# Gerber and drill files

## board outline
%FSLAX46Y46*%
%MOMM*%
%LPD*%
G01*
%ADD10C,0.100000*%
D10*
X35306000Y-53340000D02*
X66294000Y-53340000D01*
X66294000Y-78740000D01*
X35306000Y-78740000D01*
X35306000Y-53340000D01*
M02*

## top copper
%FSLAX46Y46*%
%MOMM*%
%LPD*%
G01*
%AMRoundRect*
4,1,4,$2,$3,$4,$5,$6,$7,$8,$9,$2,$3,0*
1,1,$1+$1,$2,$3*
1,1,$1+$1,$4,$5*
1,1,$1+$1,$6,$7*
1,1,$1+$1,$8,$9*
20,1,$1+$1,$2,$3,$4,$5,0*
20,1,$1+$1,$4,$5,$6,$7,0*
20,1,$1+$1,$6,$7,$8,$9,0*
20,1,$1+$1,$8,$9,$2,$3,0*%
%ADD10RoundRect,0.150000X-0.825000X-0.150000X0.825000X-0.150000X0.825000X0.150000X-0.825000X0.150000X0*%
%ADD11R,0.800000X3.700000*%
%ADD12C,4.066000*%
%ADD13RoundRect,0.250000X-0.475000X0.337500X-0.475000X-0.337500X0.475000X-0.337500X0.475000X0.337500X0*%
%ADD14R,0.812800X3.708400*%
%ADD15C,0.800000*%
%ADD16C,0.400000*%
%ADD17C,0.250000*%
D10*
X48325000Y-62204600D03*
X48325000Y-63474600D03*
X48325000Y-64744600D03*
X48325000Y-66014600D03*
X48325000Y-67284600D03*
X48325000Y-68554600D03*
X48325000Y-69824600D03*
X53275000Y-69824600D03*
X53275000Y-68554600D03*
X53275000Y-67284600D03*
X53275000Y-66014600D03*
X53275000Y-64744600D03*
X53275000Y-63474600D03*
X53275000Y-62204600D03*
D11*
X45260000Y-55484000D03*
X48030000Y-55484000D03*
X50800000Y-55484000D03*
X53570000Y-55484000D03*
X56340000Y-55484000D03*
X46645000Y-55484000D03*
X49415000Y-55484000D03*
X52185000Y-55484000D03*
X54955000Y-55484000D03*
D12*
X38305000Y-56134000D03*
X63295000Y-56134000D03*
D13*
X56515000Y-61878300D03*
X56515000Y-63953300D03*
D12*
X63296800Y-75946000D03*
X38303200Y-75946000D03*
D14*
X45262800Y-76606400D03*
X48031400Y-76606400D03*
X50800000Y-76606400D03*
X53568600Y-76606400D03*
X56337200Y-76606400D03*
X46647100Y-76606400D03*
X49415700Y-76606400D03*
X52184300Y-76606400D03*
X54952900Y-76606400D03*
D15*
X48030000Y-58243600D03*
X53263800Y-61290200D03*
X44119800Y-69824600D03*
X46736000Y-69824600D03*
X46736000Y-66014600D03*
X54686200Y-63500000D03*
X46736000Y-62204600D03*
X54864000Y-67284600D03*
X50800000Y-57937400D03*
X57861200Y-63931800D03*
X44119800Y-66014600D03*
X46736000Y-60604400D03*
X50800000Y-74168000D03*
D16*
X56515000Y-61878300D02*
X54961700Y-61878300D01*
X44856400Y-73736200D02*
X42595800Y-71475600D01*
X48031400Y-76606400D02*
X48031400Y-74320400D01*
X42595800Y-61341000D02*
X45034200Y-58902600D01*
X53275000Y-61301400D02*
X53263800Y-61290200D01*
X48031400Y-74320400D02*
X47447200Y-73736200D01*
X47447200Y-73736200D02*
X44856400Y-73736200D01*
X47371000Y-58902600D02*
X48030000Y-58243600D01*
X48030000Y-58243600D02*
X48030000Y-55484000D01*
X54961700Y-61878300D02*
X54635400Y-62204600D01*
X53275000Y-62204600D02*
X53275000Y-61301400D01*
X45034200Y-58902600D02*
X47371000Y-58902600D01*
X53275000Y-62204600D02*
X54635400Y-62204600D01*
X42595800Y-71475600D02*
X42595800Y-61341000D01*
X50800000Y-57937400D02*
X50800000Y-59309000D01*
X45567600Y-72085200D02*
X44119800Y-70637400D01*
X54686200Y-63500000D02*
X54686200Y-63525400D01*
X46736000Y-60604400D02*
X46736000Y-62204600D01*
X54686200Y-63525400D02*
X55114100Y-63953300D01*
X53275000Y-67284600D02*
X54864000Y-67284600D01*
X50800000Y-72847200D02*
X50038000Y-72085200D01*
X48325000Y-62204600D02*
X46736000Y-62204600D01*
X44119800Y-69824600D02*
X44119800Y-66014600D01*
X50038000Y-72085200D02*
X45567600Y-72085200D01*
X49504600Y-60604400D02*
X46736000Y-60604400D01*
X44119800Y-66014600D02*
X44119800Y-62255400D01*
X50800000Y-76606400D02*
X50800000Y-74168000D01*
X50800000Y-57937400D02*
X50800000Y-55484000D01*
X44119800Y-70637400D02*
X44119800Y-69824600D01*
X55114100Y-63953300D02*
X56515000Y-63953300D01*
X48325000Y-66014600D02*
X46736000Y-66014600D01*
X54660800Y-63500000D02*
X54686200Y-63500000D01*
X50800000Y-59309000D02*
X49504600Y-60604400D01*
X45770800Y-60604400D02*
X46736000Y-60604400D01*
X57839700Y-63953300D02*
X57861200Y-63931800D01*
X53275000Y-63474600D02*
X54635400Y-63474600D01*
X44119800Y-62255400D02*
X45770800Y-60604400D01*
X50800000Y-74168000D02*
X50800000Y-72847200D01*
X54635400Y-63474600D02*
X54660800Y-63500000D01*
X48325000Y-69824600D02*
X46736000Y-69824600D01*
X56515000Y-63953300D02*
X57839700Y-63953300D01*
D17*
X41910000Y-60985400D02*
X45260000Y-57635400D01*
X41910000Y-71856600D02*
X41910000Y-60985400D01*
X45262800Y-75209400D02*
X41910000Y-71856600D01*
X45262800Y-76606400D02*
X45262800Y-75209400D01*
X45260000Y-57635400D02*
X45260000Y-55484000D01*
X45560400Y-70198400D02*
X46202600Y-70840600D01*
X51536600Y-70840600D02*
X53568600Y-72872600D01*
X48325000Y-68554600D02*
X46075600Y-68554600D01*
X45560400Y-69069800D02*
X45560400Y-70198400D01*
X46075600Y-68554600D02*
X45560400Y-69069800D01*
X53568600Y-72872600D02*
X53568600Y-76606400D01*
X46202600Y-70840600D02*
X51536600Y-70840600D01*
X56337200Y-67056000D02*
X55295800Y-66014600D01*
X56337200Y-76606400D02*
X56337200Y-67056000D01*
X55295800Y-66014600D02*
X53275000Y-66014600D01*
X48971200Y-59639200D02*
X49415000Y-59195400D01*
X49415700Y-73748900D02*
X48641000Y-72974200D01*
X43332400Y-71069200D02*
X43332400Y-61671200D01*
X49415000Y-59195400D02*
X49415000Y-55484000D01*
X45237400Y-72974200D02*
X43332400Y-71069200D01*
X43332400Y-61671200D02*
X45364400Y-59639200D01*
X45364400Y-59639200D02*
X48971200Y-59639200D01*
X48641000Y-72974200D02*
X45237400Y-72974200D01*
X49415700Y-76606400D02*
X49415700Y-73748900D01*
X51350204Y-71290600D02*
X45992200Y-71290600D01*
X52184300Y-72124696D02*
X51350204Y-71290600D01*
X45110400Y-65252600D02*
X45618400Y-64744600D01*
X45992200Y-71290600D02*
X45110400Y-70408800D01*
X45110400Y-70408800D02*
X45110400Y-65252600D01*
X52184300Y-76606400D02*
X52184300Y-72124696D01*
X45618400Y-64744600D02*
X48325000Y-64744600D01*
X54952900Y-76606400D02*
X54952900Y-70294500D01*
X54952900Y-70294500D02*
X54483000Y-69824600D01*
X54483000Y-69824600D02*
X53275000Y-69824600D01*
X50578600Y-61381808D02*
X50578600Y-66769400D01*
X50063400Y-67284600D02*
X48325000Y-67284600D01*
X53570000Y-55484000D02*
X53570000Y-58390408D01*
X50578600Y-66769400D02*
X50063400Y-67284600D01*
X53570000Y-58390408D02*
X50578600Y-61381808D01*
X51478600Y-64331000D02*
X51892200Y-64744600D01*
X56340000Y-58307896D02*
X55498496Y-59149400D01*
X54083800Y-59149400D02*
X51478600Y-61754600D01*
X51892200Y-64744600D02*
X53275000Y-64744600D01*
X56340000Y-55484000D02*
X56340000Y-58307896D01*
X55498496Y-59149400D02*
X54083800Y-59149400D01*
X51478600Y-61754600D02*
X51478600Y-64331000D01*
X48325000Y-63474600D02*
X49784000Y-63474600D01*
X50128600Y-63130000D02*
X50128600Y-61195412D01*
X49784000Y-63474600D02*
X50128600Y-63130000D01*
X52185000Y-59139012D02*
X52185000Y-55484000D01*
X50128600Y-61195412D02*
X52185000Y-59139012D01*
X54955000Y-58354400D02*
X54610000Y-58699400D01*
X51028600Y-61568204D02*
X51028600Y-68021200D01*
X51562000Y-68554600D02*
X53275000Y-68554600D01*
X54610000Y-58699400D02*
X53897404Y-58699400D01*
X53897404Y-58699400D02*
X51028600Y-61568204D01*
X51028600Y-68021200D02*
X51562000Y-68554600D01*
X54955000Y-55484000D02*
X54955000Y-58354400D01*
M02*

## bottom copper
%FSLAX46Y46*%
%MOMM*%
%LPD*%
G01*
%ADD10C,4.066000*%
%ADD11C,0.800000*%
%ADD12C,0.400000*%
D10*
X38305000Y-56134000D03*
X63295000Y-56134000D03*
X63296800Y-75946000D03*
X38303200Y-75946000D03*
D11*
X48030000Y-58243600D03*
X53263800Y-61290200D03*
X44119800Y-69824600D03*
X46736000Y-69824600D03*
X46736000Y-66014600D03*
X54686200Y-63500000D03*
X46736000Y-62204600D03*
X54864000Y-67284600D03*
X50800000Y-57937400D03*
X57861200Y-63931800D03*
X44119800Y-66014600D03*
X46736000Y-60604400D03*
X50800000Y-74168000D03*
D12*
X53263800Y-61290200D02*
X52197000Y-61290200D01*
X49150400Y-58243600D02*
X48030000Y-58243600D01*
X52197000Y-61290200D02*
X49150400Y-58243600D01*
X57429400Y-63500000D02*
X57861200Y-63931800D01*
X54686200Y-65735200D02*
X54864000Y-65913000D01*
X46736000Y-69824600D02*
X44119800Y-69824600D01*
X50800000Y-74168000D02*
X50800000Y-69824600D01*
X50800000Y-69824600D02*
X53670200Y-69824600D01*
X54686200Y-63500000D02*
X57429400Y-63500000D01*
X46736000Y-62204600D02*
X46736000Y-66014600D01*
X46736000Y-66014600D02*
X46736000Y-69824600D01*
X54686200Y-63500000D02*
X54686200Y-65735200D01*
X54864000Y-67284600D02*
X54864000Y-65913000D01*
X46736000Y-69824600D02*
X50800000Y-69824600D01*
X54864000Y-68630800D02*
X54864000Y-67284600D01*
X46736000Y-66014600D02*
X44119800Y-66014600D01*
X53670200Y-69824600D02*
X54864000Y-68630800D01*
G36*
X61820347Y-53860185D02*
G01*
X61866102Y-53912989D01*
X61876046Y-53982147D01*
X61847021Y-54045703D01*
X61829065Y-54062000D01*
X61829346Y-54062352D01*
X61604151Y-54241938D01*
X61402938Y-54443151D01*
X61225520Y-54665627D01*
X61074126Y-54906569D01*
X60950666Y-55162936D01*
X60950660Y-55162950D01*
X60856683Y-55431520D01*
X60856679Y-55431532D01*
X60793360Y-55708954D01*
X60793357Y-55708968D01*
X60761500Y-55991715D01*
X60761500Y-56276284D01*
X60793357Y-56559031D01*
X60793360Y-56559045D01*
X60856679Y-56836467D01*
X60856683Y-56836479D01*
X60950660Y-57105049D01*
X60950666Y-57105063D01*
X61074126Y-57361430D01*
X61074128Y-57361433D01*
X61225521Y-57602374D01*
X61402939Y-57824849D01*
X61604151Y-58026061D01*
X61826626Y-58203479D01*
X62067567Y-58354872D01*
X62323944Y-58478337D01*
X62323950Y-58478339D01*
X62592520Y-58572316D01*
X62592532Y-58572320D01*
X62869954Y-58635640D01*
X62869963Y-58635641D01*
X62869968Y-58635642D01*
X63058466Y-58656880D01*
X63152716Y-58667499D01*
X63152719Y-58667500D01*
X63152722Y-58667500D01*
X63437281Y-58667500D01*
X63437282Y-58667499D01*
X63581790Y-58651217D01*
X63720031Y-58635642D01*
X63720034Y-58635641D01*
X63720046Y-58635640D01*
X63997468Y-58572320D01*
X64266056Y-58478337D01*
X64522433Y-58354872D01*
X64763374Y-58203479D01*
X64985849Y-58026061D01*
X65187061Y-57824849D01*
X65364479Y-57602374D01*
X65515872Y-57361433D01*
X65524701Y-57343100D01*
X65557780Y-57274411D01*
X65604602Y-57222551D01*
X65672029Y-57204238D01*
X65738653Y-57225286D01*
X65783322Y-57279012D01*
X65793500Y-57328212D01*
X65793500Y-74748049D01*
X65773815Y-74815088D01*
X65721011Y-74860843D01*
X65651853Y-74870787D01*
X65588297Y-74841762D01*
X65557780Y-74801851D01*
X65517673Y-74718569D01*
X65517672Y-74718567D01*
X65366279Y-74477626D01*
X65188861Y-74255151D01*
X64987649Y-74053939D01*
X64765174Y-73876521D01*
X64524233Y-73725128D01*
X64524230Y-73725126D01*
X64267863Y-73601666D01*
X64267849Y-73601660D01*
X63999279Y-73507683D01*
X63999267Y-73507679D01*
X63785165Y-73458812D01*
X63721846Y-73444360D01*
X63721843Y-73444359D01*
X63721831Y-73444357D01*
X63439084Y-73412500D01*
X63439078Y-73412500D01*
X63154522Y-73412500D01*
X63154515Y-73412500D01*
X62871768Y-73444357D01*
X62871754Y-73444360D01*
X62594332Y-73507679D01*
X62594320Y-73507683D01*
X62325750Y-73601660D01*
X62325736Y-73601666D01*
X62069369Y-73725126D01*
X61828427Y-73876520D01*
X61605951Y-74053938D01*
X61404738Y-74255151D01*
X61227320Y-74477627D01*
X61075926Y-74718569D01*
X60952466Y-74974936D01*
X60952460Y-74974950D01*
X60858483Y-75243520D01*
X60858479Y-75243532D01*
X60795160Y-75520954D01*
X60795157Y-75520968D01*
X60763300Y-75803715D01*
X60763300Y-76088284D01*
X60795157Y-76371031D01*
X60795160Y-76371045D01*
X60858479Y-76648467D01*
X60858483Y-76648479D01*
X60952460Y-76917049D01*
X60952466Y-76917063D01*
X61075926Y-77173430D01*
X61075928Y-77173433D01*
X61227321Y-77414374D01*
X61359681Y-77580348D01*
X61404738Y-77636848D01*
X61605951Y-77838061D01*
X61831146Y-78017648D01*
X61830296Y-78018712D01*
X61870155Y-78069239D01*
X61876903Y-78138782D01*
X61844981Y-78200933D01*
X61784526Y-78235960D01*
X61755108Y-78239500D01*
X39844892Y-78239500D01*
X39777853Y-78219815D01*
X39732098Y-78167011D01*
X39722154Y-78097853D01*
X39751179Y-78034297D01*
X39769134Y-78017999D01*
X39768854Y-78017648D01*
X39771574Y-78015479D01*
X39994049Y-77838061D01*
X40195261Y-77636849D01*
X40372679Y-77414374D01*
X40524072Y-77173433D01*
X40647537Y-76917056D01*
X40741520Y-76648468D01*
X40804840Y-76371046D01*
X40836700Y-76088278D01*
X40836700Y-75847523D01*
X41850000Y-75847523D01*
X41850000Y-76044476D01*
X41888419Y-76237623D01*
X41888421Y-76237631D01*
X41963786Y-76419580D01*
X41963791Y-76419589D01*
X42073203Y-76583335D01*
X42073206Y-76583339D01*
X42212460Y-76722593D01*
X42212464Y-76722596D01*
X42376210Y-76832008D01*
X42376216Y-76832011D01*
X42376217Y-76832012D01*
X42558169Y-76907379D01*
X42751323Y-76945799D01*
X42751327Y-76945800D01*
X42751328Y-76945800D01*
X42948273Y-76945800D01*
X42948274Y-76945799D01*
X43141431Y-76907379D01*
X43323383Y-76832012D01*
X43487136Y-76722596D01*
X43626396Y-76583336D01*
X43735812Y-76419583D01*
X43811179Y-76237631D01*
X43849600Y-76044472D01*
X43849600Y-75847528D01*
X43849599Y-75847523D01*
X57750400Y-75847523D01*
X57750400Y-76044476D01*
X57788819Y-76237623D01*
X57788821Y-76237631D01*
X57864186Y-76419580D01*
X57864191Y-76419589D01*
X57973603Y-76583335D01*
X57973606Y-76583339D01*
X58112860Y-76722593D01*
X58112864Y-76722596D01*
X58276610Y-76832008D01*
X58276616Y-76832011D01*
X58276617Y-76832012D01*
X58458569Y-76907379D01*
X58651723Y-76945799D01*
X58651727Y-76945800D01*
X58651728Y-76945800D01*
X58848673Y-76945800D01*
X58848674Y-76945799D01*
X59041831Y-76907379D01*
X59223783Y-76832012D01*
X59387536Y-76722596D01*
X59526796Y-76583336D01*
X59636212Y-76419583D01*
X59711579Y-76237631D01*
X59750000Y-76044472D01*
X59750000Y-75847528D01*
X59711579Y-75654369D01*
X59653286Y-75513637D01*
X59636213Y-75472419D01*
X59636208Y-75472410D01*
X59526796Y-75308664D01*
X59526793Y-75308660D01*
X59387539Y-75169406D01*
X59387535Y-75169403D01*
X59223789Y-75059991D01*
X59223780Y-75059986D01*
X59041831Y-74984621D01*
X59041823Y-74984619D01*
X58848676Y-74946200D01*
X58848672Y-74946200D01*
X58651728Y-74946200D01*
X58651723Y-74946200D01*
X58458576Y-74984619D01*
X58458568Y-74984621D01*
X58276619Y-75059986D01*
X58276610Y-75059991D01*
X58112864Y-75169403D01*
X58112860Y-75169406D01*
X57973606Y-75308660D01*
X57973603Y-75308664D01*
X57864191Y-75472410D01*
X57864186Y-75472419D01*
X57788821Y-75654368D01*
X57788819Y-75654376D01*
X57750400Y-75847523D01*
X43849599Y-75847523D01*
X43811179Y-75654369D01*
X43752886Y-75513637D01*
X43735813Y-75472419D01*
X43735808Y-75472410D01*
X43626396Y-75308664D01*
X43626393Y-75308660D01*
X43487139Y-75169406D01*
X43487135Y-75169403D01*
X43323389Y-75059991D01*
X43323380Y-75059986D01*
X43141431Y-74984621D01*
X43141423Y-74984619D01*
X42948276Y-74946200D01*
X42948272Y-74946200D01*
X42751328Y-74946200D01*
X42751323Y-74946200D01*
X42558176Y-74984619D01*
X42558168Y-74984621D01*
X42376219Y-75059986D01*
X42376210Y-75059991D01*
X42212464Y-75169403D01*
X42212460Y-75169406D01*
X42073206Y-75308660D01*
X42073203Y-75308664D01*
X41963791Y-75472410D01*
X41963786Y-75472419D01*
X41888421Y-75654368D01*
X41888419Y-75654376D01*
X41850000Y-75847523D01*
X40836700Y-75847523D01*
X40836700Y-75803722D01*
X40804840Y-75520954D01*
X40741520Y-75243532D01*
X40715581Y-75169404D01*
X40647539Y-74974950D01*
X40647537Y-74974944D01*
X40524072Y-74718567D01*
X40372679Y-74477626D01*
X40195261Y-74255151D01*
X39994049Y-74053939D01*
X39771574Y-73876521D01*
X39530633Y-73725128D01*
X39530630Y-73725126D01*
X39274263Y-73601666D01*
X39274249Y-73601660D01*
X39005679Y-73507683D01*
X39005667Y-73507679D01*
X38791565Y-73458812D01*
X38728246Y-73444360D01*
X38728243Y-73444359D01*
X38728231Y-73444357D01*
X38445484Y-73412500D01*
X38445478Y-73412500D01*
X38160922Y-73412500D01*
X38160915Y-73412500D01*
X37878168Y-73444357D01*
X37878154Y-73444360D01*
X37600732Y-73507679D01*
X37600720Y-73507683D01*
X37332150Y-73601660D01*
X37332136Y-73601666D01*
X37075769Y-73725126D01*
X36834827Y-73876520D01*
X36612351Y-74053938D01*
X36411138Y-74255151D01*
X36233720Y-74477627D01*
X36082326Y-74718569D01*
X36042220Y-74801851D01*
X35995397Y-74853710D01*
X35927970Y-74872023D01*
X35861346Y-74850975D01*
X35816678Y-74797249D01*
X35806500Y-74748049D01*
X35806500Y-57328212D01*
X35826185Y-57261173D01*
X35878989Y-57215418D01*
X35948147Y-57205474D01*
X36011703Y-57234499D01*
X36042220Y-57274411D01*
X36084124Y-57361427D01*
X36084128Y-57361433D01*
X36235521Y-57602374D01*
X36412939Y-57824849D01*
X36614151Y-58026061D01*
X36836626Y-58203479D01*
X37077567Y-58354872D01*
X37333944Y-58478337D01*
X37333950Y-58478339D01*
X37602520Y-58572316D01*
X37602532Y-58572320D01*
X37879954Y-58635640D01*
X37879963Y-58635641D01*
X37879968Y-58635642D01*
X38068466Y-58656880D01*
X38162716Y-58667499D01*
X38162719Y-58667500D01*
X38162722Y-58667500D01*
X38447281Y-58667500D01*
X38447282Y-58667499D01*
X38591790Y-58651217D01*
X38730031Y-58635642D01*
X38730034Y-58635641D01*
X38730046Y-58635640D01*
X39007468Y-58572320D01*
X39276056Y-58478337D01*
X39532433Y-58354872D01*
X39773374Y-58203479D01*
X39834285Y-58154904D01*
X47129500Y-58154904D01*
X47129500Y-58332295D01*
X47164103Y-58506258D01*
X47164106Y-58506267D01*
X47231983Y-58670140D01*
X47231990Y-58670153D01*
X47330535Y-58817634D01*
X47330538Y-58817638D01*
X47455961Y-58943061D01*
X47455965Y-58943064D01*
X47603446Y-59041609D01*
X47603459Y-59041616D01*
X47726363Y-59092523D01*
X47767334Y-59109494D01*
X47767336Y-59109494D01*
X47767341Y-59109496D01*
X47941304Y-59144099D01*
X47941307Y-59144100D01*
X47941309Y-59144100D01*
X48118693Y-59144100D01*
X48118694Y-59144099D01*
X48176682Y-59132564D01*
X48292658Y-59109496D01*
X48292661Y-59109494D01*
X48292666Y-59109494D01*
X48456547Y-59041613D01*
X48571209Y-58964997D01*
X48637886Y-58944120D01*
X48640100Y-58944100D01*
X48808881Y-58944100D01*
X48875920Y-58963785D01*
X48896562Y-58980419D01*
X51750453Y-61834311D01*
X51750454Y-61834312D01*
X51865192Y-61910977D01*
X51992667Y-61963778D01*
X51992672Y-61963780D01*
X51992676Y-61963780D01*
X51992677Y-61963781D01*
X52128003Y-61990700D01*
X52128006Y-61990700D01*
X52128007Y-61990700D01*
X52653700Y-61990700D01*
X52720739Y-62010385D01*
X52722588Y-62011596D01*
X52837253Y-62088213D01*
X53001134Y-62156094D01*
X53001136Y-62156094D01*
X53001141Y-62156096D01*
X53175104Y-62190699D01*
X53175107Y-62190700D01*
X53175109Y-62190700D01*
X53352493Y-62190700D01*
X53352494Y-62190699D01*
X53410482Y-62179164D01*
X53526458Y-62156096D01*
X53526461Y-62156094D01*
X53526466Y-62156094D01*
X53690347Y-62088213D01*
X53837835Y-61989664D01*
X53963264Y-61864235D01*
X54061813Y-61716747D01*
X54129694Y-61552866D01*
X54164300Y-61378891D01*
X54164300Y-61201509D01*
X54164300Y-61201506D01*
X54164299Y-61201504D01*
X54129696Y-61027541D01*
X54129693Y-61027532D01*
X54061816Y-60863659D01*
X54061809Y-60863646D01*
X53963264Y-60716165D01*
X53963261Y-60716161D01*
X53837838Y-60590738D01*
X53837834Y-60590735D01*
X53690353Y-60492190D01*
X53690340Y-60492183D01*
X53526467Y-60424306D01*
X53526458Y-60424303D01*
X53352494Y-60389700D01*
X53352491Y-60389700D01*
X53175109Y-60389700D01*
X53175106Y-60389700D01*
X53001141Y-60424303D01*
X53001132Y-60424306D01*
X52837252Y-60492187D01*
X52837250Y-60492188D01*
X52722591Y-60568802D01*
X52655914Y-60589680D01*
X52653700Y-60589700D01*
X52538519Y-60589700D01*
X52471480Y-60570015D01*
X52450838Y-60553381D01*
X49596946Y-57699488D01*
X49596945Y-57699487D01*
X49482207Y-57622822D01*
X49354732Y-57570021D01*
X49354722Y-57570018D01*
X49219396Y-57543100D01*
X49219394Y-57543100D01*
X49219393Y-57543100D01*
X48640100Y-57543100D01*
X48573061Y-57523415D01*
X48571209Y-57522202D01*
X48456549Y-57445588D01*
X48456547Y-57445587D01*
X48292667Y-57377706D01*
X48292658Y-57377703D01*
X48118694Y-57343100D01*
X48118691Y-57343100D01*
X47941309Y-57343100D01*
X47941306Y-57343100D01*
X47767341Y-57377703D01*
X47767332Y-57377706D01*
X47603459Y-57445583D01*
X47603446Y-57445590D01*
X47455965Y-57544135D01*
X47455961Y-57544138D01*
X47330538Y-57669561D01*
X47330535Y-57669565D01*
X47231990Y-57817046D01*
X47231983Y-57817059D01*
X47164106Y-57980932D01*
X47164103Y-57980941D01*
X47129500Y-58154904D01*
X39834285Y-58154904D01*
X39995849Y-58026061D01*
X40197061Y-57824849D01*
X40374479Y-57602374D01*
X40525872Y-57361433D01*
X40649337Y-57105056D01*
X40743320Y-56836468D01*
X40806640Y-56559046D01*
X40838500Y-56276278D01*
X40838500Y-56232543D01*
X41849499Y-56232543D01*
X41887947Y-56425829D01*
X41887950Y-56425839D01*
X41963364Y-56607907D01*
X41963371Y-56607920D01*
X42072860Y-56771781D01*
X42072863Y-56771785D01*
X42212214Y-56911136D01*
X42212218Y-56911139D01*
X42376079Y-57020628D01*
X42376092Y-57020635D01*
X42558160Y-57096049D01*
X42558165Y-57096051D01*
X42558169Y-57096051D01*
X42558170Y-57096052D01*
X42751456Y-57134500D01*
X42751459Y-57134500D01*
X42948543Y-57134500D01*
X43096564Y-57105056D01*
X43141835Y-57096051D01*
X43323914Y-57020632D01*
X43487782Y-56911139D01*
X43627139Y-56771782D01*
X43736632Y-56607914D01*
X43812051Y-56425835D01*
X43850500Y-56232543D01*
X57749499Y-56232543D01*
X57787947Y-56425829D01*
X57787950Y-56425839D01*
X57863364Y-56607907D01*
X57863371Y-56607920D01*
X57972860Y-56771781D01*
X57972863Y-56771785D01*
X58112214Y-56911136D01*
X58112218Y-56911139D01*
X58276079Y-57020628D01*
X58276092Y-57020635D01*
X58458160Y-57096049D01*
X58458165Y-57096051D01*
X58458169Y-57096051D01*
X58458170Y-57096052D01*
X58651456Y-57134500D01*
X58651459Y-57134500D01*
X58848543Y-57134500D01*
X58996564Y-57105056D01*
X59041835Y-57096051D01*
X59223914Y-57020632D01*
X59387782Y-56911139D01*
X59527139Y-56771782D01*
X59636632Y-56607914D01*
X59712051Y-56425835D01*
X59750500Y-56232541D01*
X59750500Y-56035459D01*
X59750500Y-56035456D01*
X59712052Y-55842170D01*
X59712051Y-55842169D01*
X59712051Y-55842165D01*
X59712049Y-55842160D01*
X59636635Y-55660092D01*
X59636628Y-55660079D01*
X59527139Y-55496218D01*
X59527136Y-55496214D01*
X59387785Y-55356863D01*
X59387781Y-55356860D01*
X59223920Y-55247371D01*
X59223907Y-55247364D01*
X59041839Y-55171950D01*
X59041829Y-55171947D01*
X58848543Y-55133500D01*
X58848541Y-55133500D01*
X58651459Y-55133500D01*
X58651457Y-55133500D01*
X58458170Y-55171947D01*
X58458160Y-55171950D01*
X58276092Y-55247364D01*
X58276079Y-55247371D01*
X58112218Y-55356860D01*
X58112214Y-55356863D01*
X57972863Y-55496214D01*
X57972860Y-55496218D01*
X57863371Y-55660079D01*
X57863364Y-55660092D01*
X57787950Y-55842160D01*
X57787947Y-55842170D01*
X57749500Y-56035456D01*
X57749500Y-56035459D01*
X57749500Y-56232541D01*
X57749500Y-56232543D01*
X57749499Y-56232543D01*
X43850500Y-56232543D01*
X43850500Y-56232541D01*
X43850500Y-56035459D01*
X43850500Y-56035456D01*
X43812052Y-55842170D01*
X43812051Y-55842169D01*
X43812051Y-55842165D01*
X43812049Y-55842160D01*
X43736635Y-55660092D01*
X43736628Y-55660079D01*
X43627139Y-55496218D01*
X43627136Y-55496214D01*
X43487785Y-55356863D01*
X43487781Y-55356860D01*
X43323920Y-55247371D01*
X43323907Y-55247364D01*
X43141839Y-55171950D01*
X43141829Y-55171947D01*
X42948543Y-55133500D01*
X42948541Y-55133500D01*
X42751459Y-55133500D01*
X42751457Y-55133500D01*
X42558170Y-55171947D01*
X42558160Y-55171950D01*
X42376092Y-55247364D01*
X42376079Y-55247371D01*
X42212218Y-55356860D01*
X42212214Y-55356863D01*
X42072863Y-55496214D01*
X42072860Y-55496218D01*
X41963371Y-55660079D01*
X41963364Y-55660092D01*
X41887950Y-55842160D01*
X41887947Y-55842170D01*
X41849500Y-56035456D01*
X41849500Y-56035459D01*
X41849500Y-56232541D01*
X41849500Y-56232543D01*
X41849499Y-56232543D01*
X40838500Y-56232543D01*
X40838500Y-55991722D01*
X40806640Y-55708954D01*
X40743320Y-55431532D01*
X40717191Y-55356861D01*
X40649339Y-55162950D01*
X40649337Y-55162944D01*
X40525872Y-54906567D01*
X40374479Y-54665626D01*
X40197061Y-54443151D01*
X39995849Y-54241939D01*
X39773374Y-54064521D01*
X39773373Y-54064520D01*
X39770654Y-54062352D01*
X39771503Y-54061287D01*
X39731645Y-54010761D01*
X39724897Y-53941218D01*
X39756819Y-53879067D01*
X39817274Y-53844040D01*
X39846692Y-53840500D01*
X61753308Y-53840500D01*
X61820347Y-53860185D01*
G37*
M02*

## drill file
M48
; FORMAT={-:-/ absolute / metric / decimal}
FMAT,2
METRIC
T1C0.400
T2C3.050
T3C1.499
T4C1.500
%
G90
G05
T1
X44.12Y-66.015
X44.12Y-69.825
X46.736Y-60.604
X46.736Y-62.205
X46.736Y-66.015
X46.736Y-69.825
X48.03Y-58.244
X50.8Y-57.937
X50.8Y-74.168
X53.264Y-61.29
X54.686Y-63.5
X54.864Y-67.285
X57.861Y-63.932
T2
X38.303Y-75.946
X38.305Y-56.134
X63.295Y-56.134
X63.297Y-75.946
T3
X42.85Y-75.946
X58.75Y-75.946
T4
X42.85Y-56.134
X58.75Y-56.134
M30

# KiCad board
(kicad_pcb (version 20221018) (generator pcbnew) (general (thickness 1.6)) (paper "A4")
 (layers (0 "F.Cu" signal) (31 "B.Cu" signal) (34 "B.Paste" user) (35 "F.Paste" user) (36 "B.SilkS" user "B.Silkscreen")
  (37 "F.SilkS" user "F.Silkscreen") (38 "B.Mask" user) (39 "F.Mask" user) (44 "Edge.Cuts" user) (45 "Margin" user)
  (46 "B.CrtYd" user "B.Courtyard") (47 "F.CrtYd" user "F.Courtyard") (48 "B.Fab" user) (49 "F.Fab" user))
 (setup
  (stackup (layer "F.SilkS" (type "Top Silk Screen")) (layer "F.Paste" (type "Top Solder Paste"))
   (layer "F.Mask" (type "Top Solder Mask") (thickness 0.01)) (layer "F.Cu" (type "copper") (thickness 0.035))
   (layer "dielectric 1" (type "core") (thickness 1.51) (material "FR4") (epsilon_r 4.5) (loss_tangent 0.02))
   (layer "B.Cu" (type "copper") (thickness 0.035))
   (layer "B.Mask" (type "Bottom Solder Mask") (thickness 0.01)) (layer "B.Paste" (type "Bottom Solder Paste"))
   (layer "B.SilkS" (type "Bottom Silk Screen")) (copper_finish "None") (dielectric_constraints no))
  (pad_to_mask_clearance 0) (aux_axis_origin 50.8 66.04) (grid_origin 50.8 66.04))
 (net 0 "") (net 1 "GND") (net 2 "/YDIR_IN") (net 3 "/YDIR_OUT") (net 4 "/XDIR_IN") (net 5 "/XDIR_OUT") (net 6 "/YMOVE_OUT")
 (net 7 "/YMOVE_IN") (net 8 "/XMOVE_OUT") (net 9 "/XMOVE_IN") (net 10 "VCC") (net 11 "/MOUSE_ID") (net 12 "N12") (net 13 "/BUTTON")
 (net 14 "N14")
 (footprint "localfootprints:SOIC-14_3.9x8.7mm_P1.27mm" (layer "F.Cu") (at 50.8 66.0146)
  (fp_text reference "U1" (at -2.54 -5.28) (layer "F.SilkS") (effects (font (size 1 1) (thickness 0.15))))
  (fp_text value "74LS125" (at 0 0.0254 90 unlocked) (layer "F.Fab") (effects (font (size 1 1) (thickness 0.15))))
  (pad "1" smd roundrect (at -2.475 -3.81) (size 1.95 0.6) (layers "F.Cu" "F.Paste" "F.Mask") (roundrect_rratio 0.25) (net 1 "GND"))
  (pad "2" smd roundrect (at -2.475 -2.54) (size 1.95 0.6) (layers "F.Cu" "F.Paste" "F.Mask") (roundrect_rratio 0.25) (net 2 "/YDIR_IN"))
  (pad "3" smd roundrect (at -2.475 -1.27) (size 1.95 0.6) (layers "F.Cu" "F.Paste" "F.Mask") (roundrect_rratio 0.25) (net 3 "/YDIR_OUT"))
  (pad "4" smd roundrect (at -2.475 0) (size 1.95 0.6) (layers "F.Cu" "F.Paste" "F.Mask") (roundrect_rratio 0.25) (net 1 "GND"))
  (pad "5" smd roundrect (at -2.475 1.27) (size 1.95 0.6) (layers "F.Cu" "F.Paste" "F.Mask") (roundrect_rratio 0.25) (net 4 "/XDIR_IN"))
  (pad "6" smd roundrect (at -2.475 2.54) (size 1.95 0.6) (layers "F.Cu" "F.Paste" "F.Mask") (roundrect_rratio 0.25) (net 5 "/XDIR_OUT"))
  (pad "7" smd roundrect (at -2.475 3.81) (size 1.95 0.6) (layers "F.Cu" "F.Paste" "F.Mask") (roundrect_rratio 0.25) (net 1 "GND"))
  (pad "8" smd roundrect (at 2.475 3.81) (size 1.95 0.6) (layers "F.Cu" "F.Paste" "F.Mask") (roundrect_rratio 0.25) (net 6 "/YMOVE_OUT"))
  (pad "9" smd roundrect (at 2.475 2.54) (size 1.95 0.6) (layers "F.Cu" "F.Paste" "F.Mask") (roundrect_rratio 0.25) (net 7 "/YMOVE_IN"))
  (pad "10" smd roundrect (at 2.475 1.27) (size 1.95 0.6) (layers "F.Cu" "F.Paste" "F.Mask") (roundrect_rratio 0.25) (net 1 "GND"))
  (pad "11" smd roundrect (at 2.475 0) (size 1.95 0.6) (layers "F.Cu" "F.Paste" "F.Mask") (roundrect_rratio 0.25) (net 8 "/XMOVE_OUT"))
  (pad "12" smd roundrect (at 2.475 -1.27) (size 1.95 0.6) (layers "F.Cu" "F.Paste" "F.Mask") (roundrect_rratio 0.25) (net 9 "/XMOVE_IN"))
  (pad "13" smd roundrect (at 2.475 -2.54) (size 1.95 0.6) (layers "F.Cu" "F.Paste" "F.Mask") (roundrect_rratio 0.25) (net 1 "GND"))
  (pad "14" smd roundrect (at 2.475 -3.81) (size 1.95 0.6) (layers "F.Cu" "F.Paste" "F.Mask") (roundrect_rratio 0.25) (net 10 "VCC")))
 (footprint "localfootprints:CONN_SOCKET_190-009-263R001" (layer "F.Cu") (at 50.8 56.134)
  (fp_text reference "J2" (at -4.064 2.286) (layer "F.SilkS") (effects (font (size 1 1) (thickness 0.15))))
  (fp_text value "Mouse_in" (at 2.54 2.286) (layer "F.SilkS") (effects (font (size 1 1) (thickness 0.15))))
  (pad "" np_thru_hole circle (at -7.95 0) (size 1.5 1.5) (drill 1.5) (layers "*.Cu" "*.Mask"))
  (pad "" np_thru_hole circle (at 7.95 0) (size 1.5 1.5) (drill 1.5) (layers "*.Cu" "*.Mask"))
  (pad "1" smd rect (at -5.54 -0.65) (size 0.8 3.7) (layers "F.Cu" "F.Paste" "F.Mask") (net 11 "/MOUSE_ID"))
  (pad "2" smd rect (at -2.77 -0.65) (size 0.8 3.7) (layers "F.Cu" "F.Paste" "F.Mask") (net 10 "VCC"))
  (pad "3" smd rect (at 0 -0.65) (size 0.8 3.7) (layers "F.Cu" "F.Paste" "F.Mask") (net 1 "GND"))
  (pad "4" smd rect (at 2.77 -0.65) (size 0.8 3.7) (layers "F.Cu" "F.Paste" "F.Mask") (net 4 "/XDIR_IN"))
  (pad "5" smd rect (at 5.54 -0.65) (size 0.8 3.7) (layers "F.Cu" "F.Paste" "F.Mask") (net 9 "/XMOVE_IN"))
  (pad "6" smd rect (at -4.155 -0.65) (size 0.8 3.7) (layers "F.Cu" "F.Paste" "F.Mask") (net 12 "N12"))
  (pad "7" smd rect (at -1.385 -0.65) (size 0.8 3.7) (layers "F.Cu" "F.Paste" "F.Mask") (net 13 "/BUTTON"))
  (pad "8" smd rect (at 1.385 -0.65) (size 0.8 3.7) (layers "F.Cu" "F.Paste" "F.Mask") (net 2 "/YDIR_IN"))
  (pad "9" smd rect (at 4.155 -0.65) (size 0.8 3.7) (layers "F.Cu" "F.Paste" "F.Mask") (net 7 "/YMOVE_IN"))
  (pad "S1" thru_hole circle (at -12.495 0) (size 4.066 4.066) (drill 3.05) (layers "*.Cu" "*.Mask"))
  (pad "S2" thru_hole circle (at 12.495 0) (size 4.066 4.066) (drill 3.05) (layers "*.Cu" "*.Mask")))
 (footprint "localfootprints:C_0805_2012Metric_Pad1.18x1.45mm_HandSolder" (layer "F.Cu") (at 56.515 62.9158 -90)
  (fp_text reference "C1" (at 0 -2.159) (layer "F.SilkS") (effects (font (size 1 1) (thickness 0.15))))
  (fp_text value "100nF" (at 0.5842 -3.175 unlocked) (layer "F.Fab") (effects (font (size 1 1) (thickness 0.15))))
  (pad "1" smd roundrect (at -1.0375 0 270) (size 1.175 1.45) (layers "F.Cu" "F.Paste" "F.Mask") (roundrect_rratio 0.2127659574)
   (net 10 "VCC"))
  (pad "2" smd roundrect (at 1.0375 0 270) (size 1.175 1.45) (layers "F.Cu" "F.Paste" "F.Mask") (roundrect_rratio 0.2127659574)
   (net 1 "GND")))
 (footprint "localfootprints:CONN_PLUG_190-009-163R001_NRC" (layer "F.Cu") (at 50.8 75.946 180)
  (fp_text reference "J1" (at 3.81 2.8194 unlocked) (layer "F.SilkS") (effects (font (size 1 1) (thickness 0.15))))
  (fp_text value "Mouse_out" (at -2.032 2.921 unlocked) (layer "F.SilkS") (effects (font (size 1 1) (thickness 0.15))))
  (pad "" thru_hole circle (at -12.4968 0 180) (size 4.066 4.066) (drill 3.05) (layers "*.Cu" "*.Mask"))
  (pad "" np_thru_hole circle (at -7.9502 0 180) (size 1.4986 1.4986) (drill 1.4986) (layers))
  (pad "" np_thru_hole circle (at 7.9502 0 180) (size 1.4986 1.4986) (drill 1.4986) (layers))
  (pad "" thru_hole circle (at 12.4968 0 180) (size 4.066 4.066) (drill 3.05) (layers "*.Cu" "*.Mask"))
  (pad "1" smd rect (at 5.5372 -0.6604 180) (size 0.8128 3.7084) (layers "F.Cu" "F.Paste" "F.Mask") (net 11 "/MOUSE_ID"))
  (pad "2" smd rect (at 2.7686 -0.6604 180) (size 0.8128 3.7084) (layers "F.Cu" "F.Paste" "F.Mask") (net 10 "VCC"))
  (pad "3" smd rect (at 0 -0.6604 180) (size 0.8128 3.7084) (layers "F.Cu" "F.Paste" "F.Mask") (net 1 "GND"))
  (pad "4" smd rect (at -2.7686 -0.6604 180) (size 0.8128 3.7084) (layers "F.Cu" "F.Paste" "F.Mask") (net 5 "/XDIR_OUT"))
  (pad "5" smd rect (at -5.5372 -0.6604 180) (size 0.8128 3.7084) (layers "F.Cu" "F.Paste" "F.Mask") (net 8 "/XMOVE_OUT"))
  (pad "6" smd rect (at 4.1529 -0.6604 180) (size 0.8128 3.7084) (layers "F.Cu" "F.Paste" "F.Mask") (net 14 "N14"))
  (pad "7" smd rect (at 1.3843 -0.6604 180) (size 0.8128 3.7084) (layers "F.Cu" "F.Paste" "F.Mask") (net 13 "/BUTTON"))
  (pad "8" smd rect (at -1.3843 -0.6604 180) (size 0.8128 3.7084) (layers "F.Cu" "F.Paste" "F.Mask") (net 3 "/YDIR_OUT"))
  (pad "9" smd rect (at -4.1529 -0.6604 180) (size 0.8128 3.7084) (layers "F.Cu" "F.Paste" "F.Mask") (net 6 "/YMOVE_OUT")))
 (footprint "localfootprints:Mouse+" (layer "B.Cu") (at 50.8 66.04 180)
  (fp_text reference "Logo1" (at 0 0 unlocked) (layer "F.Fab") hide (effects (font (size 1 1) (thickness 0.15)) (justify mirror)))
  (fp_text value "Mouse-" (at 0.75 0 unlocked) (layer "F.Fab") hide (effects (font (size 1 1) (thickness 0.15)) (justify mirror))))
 (gr_rect (start 35.306 53.34) (end 66.294 78.74) (stroke (width 0.1) (type default)) (fill none) (layer "Edge.Cuts"))
 (segment (start 56.515 61.8783) (end 54.9617 61.8783) (width 0.4) (layer "F.Cu") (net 10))
 (segment (start 44.8564 73.7362) (end 42.5958 71.4756) (width 0.4) (layer "F.Cu") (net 10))
 (segment (start 48.0314 76.6064) (end 48.0314 74.3204) (width 0.4) (layer "F.Cu") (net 10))
 (segment (start 42.5958 61.341) (end 45.0342 58.9026) (width 0.4) (layer "F.Cu") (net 10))
 (segment (start 53.275 61.3014) (end 53.2638 61.2902) (width 0.4) (layer "F.Cu") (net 10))
 (segment (start 48.0314 74.3204) (end 47.4472 73.7362) (width 0.4) (layer "F.Cu") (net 10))
 (segment (start 47.4472 73.7362) (end 44.8564 73.7362) (width 0.4) (layer "F.Cu") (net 10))
 (segment (start 47.371 58.9026) (end 48.03 58.2436) (width 0.4) (layer "F.Cu") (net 10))
 (segment (start 48.03 58.2436) (end 48.03 55.484) (width 0.4) (layer "F.Cu") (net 10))
 (segment (start 54.9617 61.8783) (end 54.6354 62.2046) (width 0.4) (layer "F.Cu") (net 10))
 (segment (start 53.275 62.2046) (end 53.275 61.3014) (width 0.4) (layer "F.Cu") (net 10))
 (segment (start 45.0342 58.9026) (end 47.371 58.9026) (width 0.4) (layer "F.Cu") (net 10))
 (segment (start 53.275 62.2046) (end 54.6354 62.2046) (width 0.4) (layer "F.Cu") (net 10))
 (segment (start 42.5958 71.4756) (end 42.5958 61.341) (width 0.4) (layer "F.Cu") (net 10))
 (via (at 48.03 58.2436) (size 0.8) (drill 0.4) (layers "F.Cu" "B.Cu") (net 10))
 (via (at 53.2638 61.2902) (size 0.8) (drill 0.4) (layers "F.Cu" "B.Cu") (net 10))
 (segment (start 53.2638 61.2902) (end 52.197 61.2902) (width 0.4) (layer "B.Cu") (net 10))
 (segment (start 49.1504 58.2436) (end 48.03 58.2436) (width 0.4) (layer "B.Cu") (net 10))
 (segment (start 52.197 61.2902) (end 49.1504 58.2436) (width 0.4) (layer "B.Cu") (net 10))
 (segment (start 50.8 57.9374) (end 50.8 59.309) (width 0.4) (layer "F.Cu") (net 1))
 (segment (start 45.5676 72.0852) (end 44.1198 70.6374) (width 0.4) (layer "F.Cu") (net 1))
 (segment (start 54.6862 63.5) (end 54.6862 63.5254) (width 0.4) (layer "F.Cu") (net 1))
 (segment (start 46.736 60.6044) (end 46.736 62.2046) (width 0.4) (layer "F.Cu") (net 1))
 (segment (start 54.6862 63.5254) (end 55.1141 63.9533) (width 0.4) (layer "F.Cu") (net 1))
 (segment (start 53.275 67.2846) (end 54.864 67.2846) (width 0.4) (layer "F.Cu") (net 1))
 (segment (start 50.8 72.8472) (end 50.038 72.0852) (width 0.4) (layer "F.Cu") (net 1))
 (segment (start 48.325 62.2046) (end 46.736 62.2046) (width 0.4) (layer "F.Cu") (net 1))
 (segment (start 44.1198 69.8246) (end 44.1198 66.0146) (width 0.4) (layer "F.Cu") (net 1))
 (segment (start 50.038 72.0852) (end 45.5676 72.0852) (width 0.4) (layer "F.Cu") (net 1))
 (segment (start 49.5046 60.6044) (end 46.736 60.6044) (width 0.4) (layer "F.Cu") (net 1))
 (segment (start 44.1198 66.0146) (end 44.1198 62.2554) (width 0.4) (layer "F.Cu") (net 1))
 (segment (start 50.8 76.6064) (end 50.8 74.168) (width 0.4) (layer "F.Cu") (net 1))
 (segment (start 50.8 57.9374) (end 50.8 55.484) (width 0.4) (layer "F.Cu") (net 1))
 (segment (start 44.1198 70.6374) (end 44.1198 69.8246) (width 0.4) (layer "F.Cu") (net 1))
 (segment (start 55.1141 63.9533) (end 56.515 63.9533) (width 0.4) (layer "F.Cu") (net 1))
 (segment (start 48.325 66.0146) (end 46.736 66.0146) (width 0.4) (layer "F.Cu") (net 1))
 (segment (start 54.6608 63.5) (end 54.6862 63.5) (width 0.4) (layer "F.Cu") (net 1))
 (segment (start 50.8 59.309) (end 49.5046 60.6044) (width 0.4) (layer "F.Cu") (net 1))
 (segment (start 45.7708 60.6044) (end 46.736 60.6044) (width 0.4) (layer "F.Cu") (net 1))
 (segment (start 57.8397 63.9533) (end 57.8612 63.9318) (width 0.4) (layer "F.Cu") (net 1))
 (segment (start 53.275 63.4746) (end 54.6354 63.4746) (width 0.4) (layer "F.Cu") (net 1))
 (segment (start 44.1198 62.2554) (end 45.7708 60.6044) (width 0.4) (layer "F.Cu") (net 1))
 (segment (start 50.8 74.168) (end 50.8 72.8472) (width 0.4) (layer "F.Cu") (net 1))
 (segment (start 54.6354 63.4746) (end 54.6608 63.5) (width 0.4) (layer "F.Cu") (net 1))
 (segment (start 48.325 69.8246) (end 46.736 69.8246) (width 0.4) (layer "F.Cu") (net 1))
 (segment (start 56.515 63.9533) (end 57.8397 63.9533) (width 0.4) (layer "F.Cu") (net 1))
 (via (at 44.1198 69.8246) (size 0.8) (drill 0.4) (layers "F.Cu" "B.Cu") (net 1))
 (via (at 46.736 69.8246) (size 0.8) (drill 0.4) (layers "F.Cu" "B.Cu") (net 1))
 (via (at 46.736 66.0146) (size 0.8) (drill 0.4) (layers "F.Cu" "B.Cu") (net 1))
 (via (at 54.6862 63.5) (size 0.8) (drill 0.4) (layers "F.Cu" "B.Cu") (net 1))
 (via (at 46.736 62.2046) (size 0.8) (drill 0.4) (layers "F.Cu" "B.Cu") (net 1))
 (via (at 54.864 67.2846) (size 0.8) (drill 0.4) (layers "F.Cu" "B.Cu") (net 1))
 (via (at 50.8 57.9374) (size 0.8) (drill 0.4) (layers "F.Cu" "B.Cu") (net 1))
 (via (at 57.8612 63.9318) (size 0.8) (drill 0.4) (layers "F.Cu" "B.Cu") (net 1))
 (via (at 44.1198 66.0146) (size 0.8) (drill 0.4) (layers "F.Cu" "B.Cu") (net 1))
 (via (at 46.736 60.6044) (size 0.8) (drill 0.4) (layers "F.Cu" "B.Cu") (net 1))
 (via (at 50.8 74.168) (size 0.8) (drill 0.4) (layers "F.Cu" "B.Cu") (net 1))
 (segment (start 57.4294 63.5) (end 57.8612 63.9318) (width 0.4) (layer "B.Cu") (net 1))
 (segment (start 54.6862 65.7352) (end 54.864 65.913) (width 0.4) (layer "B.Cu") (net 1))
 (segment (start 46.736 69.8246) (end 44.1198 69.8246) (width 0.4) (layer "B.Cu") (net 1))
 (segment (start 50.8 74.168) (end 50.8 69.8246) (width 0.4) (layer "B.Cu") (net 1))
 (segment (start 50.8 69.8246) (end 53.6702 69.8246) (width 0.4) (layer "B.Cu") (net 1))
 (segment (start 54.6862 63.5) (end 57.4294 63.5) (width 0.4) (layer "B.Cu") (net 1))
 (segment (start 46.736 62.2046) (end 46.736 66.0146) (width 0.4) (layer "B.Cu") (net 1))
 (segment (start 46.736 66.0146) (end 46.736 69.8246) (width 0.4) (layer "B.Cu") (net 1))
 (segment (start 54.6862 63.5) (end 54.6862 65.7352) (width 0.4) (layer "B.Cu") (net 1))
 (segment (start 54.864 67.2846) (end 54.864 65.913) (width 0.4) (layer "B.Cu") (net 1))
 (segment (start 46.736 69.8246) (end 50.8 69.8246) (width 0.4) (layer "B.Cu") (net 1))
 (segment (start 54.864 68.6308) (end 54.864 67.2846) (width 0.4) (layer "B.Cu") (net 1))
 (segment (start 46.736 66.0146) (end 44.1198 66.0146) (width 0.4) (layer "B.Cu") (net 1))
 (segment (start 53.6702 69.8246) (end 54.864 68.6308) (width 0.4) (layer "B.Cu") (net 1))
 (segment (start 41.91 60.9854) (end 45.26 57.6354) (width 0.25) (layer "F.Cu") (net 11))
 (segment (start 41.91 71.8566) (end 41.91 60.9854) (width 0.25) (layer "F.Cu") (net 11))
 (segment (start 45.2628 75.2094) (end 41.91 71.8566) (width 0.25) (layer "F.Cu") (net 11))
 (segment (start 45.2628 76.6064) (end 45.2628 75.2094) (width 0.25) (layer "F.Cu") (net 11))
 (segment (start 45.26 57.6354) (end 45.26 55.484) (width 0.25) (layer "F.Cu") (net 11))
 (segment (start 45.5604 70.1984) (end 46.2026 70.8406) (width 0.25) (layer "F.Cu") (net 5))
 (segment (start 51.5366 70.8406) (end 53.5686 72.8726) (width 0.25) (layer "F.Cu") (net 5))
 (segment (start 48.325 68.5546) (end 46.0756 68.5546) (width 0.25) (layer "F.Cu") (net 5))
 (segment (start 45.5604 69.0698) (end 45.5604 70.1984) (width 0.25) (layer "F.Cu") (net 5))
 (segment (start 46.0756 68.5546) (end 45.5604 69.0698) (width 0.25) (layer "F.Cu") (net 5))
 (segment (start 53.5686 72.8726) (end 53.5686 76.6064) (width 0.25) (layer "F.Cu") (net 5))
 (segment (start 46.2026 70.8406) (end 51.5366 70.8406) (width 0.25) (layer "F.Cu") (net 5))
 (segment (start 56.3372 67.056) (end 55.2958 66.0146) (width 0.25) (layer "F.Cu") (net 8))
 (segment (start 56.3372 76.6064) (end 56.3372 67.056) (width 0.25) (layer "F.Cu") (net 8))
 (segment (start 55.2958 66.0146) (end 53.275 66.0146) (width 0.25) (layer "F.Cu") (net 8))
 (segment (start 48.9712 59.6392) (end 49.415 59.1954) (width 0.25) (layer "F.Cu") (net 13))
 (segment (start 49.4157 73.7489) (end 48.641 72.9742) (width 0.25) (layer "F.Cu") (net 13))
 (segment (start 43.3324 71.0692) (end 43.3324 61.6712) (width 0.25) (layer "F.Cu") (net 13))
 (segment (start 49.415 59.1954) (end 49.415 55.484) (width 0.25) (layer "F.Cu") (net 13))
 (segment (start 45.2374 72.9742) (end 43.3324 71.0692) (width 0.25) (layer "F.Cu") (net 13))
 (segment (start 43.3324 61.6712) (end 45.3644 59.6392) (width 0.25) (layer "F.Cu") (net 13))
 (segment (start 45.3644 59.6392) (end 48.9712 59.6392) (width 0.25) (layer "F.Cu") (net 13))
 (segment (start 48.641 72.9742) (end 45.2374 72.9742) (width 0.25) (layer "F.Cu") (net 13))
 (segment (start 49.4157 76.6064) (end 49.4157 73.7489) (width 0.25) (layer "F.Cu") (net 13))
 (segment (start 51.350204 71.2906) (end 45.9922 71.2906) (width 0.25) (layer "F.Cu") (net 3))
 (segment (start 52.1843 72.124696) (end 51.350204 71.2906) (width 0.25) (layer "F.Cu") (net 3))
 (segment (start 45.1104 65.2526) (end 45.6184 64.7446) (width 0.25) (layer "F.Cu") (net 3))
 (segment (start 45.9922 71.2906) (end 45.1104 70.4088) (width 0.25) (layer "F.Cu") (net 3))
 (segment (start 45.1104 70.4088) (end 45.1104 65.2526) (width 0.25) (layer "F.Cu") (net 3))
 (segment (start 52.1843 76.6064) (end 52.1843 72.124696) (width 0.25) (layer "F.Cu") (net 3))
 (segment (start 45.6184 64.7446) (end 48.325 64.7446) (width 0.25) (layer "F.Cu") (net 3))
 (segment (start 54.9529 76.6064) (end 54.9529 70.2945) (width 0.25) (layer "F.Cu") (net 6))
 (segment (start 54.9529 70.2945) (end 54.483 69.8246) (width 0.25) (layer "F.Cu") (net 6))
 (segment (start 54.483 69.8246) (end 53.275 69.8246) (width 0.25) (layer "F.Cu") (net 6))
 (segment (start 50.5786 61.381808) (end 50.5786 66.7694) (width 0.25) (layer "F.Cu") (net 4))
 (segment (start 50.0634 67.2846) (end 48.325 67.2846) (width 0.25) (layer "F.Cu") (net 4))
 (segment (start 53.57 55.484) (end 53.57 58.390408) (width 0.25) (layer "F.Cu") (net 4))
 (segment (start 50.5786 66.7694) (end 50.0634 67.2846) (width 0.25) (layer "F.Cu") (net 4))
 (segment (start 53.57 58.390408) (end 50.5786 61.381808) (width 0.25) (layer "F.Cu") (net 4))
 (segment (start 51.4786 64.331) (end 51.8922 64.7446) (width 0.25) (layer "F.Cu") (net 9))
 (segment (start 56.34 58.307896) (end 55.498496 59.1494) (width 0.25) (layer "F.Cu") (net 9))
 (segment (start 54.0838 59.1494) (end 51.4786 61.7546) (width 0.25) (layer "F.Cu") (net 9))
 (segment (start 51.8922 64.7446) (end 53.275 64.7446) (width 0.25) (layer "F.Cu") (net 9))
 (segment (start 56.34 55.484) (end 56.34 58.307896) (width 0.25) (layer "F.Cu") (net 9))
 (segment (start 55.498496 59.1494) (end 54.0838 59.1494) (width 0.25) (layer "F.Cu") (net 9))
 (segment (start 51.4786 61.7546) (end 51.4786 64.331) (width 0.25) (layer "F.Cu") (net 9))
 (segment (start 48.325 63.4746) (end 49.784 63.4746) (width 0.25) (layer "F.Cu") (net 2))
 (segment (start 50.1286 63.13) (end 50.1286 61.195412) (width 0.25) (layer "F.Cu") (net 2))
 (segment (start 49.784 63.4746) (end 50.1286 63.13) (width 0.25) (layer "F.Cu") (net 2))
 (segment (start 52.185 59.139012) (end 52.185 55.484) (width 0.25) (layer "F.Cu") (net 2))
 (segment (start 50.1286 61.195412) (end 52.185 59.139012) (width 0.25) (layer "F.Cu") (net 2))
 (segment (start 54.955 58.3544) (end 54.61 58.6994) (width 0.25) (layer "F.Cu") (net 7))
 (segment (start 51.0286 61.568204) (end 51.0286 68.0212) (width 0.25) (layer "F.Cu") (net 7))
 (segment (start 51.562 68.5546) (end 53.275 68.5546) (width 0.25) (layer "F.Cu") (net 7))
 (segment (start 54.61 58.6994) (end 53.897404 58.6994) (width 0.25) (layer "F.Cu") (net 7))
 (segment (start 53.897404 58.6994) (end 51.0286 61.568204) (width 0.25) (layer "F.Cu") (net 7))
 (segment (start 51.0286 68.0212) (end 51.562 68.5546) (width 0.25) (layer "F.Cu") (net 7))
 (segment (start 54.955 55.484) (end 54.955 58.3544) (width 0.25) (layer "F.Cu") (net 7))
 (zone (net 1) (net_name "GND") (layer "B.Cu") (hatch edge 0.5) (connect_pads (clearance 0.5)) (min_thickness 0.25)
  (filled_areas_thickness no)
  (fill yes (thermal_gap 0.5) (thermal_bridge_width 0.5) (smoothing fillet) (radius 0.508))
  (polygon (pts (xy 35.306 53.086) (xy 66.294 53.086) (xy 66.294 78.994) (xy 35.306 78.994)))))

